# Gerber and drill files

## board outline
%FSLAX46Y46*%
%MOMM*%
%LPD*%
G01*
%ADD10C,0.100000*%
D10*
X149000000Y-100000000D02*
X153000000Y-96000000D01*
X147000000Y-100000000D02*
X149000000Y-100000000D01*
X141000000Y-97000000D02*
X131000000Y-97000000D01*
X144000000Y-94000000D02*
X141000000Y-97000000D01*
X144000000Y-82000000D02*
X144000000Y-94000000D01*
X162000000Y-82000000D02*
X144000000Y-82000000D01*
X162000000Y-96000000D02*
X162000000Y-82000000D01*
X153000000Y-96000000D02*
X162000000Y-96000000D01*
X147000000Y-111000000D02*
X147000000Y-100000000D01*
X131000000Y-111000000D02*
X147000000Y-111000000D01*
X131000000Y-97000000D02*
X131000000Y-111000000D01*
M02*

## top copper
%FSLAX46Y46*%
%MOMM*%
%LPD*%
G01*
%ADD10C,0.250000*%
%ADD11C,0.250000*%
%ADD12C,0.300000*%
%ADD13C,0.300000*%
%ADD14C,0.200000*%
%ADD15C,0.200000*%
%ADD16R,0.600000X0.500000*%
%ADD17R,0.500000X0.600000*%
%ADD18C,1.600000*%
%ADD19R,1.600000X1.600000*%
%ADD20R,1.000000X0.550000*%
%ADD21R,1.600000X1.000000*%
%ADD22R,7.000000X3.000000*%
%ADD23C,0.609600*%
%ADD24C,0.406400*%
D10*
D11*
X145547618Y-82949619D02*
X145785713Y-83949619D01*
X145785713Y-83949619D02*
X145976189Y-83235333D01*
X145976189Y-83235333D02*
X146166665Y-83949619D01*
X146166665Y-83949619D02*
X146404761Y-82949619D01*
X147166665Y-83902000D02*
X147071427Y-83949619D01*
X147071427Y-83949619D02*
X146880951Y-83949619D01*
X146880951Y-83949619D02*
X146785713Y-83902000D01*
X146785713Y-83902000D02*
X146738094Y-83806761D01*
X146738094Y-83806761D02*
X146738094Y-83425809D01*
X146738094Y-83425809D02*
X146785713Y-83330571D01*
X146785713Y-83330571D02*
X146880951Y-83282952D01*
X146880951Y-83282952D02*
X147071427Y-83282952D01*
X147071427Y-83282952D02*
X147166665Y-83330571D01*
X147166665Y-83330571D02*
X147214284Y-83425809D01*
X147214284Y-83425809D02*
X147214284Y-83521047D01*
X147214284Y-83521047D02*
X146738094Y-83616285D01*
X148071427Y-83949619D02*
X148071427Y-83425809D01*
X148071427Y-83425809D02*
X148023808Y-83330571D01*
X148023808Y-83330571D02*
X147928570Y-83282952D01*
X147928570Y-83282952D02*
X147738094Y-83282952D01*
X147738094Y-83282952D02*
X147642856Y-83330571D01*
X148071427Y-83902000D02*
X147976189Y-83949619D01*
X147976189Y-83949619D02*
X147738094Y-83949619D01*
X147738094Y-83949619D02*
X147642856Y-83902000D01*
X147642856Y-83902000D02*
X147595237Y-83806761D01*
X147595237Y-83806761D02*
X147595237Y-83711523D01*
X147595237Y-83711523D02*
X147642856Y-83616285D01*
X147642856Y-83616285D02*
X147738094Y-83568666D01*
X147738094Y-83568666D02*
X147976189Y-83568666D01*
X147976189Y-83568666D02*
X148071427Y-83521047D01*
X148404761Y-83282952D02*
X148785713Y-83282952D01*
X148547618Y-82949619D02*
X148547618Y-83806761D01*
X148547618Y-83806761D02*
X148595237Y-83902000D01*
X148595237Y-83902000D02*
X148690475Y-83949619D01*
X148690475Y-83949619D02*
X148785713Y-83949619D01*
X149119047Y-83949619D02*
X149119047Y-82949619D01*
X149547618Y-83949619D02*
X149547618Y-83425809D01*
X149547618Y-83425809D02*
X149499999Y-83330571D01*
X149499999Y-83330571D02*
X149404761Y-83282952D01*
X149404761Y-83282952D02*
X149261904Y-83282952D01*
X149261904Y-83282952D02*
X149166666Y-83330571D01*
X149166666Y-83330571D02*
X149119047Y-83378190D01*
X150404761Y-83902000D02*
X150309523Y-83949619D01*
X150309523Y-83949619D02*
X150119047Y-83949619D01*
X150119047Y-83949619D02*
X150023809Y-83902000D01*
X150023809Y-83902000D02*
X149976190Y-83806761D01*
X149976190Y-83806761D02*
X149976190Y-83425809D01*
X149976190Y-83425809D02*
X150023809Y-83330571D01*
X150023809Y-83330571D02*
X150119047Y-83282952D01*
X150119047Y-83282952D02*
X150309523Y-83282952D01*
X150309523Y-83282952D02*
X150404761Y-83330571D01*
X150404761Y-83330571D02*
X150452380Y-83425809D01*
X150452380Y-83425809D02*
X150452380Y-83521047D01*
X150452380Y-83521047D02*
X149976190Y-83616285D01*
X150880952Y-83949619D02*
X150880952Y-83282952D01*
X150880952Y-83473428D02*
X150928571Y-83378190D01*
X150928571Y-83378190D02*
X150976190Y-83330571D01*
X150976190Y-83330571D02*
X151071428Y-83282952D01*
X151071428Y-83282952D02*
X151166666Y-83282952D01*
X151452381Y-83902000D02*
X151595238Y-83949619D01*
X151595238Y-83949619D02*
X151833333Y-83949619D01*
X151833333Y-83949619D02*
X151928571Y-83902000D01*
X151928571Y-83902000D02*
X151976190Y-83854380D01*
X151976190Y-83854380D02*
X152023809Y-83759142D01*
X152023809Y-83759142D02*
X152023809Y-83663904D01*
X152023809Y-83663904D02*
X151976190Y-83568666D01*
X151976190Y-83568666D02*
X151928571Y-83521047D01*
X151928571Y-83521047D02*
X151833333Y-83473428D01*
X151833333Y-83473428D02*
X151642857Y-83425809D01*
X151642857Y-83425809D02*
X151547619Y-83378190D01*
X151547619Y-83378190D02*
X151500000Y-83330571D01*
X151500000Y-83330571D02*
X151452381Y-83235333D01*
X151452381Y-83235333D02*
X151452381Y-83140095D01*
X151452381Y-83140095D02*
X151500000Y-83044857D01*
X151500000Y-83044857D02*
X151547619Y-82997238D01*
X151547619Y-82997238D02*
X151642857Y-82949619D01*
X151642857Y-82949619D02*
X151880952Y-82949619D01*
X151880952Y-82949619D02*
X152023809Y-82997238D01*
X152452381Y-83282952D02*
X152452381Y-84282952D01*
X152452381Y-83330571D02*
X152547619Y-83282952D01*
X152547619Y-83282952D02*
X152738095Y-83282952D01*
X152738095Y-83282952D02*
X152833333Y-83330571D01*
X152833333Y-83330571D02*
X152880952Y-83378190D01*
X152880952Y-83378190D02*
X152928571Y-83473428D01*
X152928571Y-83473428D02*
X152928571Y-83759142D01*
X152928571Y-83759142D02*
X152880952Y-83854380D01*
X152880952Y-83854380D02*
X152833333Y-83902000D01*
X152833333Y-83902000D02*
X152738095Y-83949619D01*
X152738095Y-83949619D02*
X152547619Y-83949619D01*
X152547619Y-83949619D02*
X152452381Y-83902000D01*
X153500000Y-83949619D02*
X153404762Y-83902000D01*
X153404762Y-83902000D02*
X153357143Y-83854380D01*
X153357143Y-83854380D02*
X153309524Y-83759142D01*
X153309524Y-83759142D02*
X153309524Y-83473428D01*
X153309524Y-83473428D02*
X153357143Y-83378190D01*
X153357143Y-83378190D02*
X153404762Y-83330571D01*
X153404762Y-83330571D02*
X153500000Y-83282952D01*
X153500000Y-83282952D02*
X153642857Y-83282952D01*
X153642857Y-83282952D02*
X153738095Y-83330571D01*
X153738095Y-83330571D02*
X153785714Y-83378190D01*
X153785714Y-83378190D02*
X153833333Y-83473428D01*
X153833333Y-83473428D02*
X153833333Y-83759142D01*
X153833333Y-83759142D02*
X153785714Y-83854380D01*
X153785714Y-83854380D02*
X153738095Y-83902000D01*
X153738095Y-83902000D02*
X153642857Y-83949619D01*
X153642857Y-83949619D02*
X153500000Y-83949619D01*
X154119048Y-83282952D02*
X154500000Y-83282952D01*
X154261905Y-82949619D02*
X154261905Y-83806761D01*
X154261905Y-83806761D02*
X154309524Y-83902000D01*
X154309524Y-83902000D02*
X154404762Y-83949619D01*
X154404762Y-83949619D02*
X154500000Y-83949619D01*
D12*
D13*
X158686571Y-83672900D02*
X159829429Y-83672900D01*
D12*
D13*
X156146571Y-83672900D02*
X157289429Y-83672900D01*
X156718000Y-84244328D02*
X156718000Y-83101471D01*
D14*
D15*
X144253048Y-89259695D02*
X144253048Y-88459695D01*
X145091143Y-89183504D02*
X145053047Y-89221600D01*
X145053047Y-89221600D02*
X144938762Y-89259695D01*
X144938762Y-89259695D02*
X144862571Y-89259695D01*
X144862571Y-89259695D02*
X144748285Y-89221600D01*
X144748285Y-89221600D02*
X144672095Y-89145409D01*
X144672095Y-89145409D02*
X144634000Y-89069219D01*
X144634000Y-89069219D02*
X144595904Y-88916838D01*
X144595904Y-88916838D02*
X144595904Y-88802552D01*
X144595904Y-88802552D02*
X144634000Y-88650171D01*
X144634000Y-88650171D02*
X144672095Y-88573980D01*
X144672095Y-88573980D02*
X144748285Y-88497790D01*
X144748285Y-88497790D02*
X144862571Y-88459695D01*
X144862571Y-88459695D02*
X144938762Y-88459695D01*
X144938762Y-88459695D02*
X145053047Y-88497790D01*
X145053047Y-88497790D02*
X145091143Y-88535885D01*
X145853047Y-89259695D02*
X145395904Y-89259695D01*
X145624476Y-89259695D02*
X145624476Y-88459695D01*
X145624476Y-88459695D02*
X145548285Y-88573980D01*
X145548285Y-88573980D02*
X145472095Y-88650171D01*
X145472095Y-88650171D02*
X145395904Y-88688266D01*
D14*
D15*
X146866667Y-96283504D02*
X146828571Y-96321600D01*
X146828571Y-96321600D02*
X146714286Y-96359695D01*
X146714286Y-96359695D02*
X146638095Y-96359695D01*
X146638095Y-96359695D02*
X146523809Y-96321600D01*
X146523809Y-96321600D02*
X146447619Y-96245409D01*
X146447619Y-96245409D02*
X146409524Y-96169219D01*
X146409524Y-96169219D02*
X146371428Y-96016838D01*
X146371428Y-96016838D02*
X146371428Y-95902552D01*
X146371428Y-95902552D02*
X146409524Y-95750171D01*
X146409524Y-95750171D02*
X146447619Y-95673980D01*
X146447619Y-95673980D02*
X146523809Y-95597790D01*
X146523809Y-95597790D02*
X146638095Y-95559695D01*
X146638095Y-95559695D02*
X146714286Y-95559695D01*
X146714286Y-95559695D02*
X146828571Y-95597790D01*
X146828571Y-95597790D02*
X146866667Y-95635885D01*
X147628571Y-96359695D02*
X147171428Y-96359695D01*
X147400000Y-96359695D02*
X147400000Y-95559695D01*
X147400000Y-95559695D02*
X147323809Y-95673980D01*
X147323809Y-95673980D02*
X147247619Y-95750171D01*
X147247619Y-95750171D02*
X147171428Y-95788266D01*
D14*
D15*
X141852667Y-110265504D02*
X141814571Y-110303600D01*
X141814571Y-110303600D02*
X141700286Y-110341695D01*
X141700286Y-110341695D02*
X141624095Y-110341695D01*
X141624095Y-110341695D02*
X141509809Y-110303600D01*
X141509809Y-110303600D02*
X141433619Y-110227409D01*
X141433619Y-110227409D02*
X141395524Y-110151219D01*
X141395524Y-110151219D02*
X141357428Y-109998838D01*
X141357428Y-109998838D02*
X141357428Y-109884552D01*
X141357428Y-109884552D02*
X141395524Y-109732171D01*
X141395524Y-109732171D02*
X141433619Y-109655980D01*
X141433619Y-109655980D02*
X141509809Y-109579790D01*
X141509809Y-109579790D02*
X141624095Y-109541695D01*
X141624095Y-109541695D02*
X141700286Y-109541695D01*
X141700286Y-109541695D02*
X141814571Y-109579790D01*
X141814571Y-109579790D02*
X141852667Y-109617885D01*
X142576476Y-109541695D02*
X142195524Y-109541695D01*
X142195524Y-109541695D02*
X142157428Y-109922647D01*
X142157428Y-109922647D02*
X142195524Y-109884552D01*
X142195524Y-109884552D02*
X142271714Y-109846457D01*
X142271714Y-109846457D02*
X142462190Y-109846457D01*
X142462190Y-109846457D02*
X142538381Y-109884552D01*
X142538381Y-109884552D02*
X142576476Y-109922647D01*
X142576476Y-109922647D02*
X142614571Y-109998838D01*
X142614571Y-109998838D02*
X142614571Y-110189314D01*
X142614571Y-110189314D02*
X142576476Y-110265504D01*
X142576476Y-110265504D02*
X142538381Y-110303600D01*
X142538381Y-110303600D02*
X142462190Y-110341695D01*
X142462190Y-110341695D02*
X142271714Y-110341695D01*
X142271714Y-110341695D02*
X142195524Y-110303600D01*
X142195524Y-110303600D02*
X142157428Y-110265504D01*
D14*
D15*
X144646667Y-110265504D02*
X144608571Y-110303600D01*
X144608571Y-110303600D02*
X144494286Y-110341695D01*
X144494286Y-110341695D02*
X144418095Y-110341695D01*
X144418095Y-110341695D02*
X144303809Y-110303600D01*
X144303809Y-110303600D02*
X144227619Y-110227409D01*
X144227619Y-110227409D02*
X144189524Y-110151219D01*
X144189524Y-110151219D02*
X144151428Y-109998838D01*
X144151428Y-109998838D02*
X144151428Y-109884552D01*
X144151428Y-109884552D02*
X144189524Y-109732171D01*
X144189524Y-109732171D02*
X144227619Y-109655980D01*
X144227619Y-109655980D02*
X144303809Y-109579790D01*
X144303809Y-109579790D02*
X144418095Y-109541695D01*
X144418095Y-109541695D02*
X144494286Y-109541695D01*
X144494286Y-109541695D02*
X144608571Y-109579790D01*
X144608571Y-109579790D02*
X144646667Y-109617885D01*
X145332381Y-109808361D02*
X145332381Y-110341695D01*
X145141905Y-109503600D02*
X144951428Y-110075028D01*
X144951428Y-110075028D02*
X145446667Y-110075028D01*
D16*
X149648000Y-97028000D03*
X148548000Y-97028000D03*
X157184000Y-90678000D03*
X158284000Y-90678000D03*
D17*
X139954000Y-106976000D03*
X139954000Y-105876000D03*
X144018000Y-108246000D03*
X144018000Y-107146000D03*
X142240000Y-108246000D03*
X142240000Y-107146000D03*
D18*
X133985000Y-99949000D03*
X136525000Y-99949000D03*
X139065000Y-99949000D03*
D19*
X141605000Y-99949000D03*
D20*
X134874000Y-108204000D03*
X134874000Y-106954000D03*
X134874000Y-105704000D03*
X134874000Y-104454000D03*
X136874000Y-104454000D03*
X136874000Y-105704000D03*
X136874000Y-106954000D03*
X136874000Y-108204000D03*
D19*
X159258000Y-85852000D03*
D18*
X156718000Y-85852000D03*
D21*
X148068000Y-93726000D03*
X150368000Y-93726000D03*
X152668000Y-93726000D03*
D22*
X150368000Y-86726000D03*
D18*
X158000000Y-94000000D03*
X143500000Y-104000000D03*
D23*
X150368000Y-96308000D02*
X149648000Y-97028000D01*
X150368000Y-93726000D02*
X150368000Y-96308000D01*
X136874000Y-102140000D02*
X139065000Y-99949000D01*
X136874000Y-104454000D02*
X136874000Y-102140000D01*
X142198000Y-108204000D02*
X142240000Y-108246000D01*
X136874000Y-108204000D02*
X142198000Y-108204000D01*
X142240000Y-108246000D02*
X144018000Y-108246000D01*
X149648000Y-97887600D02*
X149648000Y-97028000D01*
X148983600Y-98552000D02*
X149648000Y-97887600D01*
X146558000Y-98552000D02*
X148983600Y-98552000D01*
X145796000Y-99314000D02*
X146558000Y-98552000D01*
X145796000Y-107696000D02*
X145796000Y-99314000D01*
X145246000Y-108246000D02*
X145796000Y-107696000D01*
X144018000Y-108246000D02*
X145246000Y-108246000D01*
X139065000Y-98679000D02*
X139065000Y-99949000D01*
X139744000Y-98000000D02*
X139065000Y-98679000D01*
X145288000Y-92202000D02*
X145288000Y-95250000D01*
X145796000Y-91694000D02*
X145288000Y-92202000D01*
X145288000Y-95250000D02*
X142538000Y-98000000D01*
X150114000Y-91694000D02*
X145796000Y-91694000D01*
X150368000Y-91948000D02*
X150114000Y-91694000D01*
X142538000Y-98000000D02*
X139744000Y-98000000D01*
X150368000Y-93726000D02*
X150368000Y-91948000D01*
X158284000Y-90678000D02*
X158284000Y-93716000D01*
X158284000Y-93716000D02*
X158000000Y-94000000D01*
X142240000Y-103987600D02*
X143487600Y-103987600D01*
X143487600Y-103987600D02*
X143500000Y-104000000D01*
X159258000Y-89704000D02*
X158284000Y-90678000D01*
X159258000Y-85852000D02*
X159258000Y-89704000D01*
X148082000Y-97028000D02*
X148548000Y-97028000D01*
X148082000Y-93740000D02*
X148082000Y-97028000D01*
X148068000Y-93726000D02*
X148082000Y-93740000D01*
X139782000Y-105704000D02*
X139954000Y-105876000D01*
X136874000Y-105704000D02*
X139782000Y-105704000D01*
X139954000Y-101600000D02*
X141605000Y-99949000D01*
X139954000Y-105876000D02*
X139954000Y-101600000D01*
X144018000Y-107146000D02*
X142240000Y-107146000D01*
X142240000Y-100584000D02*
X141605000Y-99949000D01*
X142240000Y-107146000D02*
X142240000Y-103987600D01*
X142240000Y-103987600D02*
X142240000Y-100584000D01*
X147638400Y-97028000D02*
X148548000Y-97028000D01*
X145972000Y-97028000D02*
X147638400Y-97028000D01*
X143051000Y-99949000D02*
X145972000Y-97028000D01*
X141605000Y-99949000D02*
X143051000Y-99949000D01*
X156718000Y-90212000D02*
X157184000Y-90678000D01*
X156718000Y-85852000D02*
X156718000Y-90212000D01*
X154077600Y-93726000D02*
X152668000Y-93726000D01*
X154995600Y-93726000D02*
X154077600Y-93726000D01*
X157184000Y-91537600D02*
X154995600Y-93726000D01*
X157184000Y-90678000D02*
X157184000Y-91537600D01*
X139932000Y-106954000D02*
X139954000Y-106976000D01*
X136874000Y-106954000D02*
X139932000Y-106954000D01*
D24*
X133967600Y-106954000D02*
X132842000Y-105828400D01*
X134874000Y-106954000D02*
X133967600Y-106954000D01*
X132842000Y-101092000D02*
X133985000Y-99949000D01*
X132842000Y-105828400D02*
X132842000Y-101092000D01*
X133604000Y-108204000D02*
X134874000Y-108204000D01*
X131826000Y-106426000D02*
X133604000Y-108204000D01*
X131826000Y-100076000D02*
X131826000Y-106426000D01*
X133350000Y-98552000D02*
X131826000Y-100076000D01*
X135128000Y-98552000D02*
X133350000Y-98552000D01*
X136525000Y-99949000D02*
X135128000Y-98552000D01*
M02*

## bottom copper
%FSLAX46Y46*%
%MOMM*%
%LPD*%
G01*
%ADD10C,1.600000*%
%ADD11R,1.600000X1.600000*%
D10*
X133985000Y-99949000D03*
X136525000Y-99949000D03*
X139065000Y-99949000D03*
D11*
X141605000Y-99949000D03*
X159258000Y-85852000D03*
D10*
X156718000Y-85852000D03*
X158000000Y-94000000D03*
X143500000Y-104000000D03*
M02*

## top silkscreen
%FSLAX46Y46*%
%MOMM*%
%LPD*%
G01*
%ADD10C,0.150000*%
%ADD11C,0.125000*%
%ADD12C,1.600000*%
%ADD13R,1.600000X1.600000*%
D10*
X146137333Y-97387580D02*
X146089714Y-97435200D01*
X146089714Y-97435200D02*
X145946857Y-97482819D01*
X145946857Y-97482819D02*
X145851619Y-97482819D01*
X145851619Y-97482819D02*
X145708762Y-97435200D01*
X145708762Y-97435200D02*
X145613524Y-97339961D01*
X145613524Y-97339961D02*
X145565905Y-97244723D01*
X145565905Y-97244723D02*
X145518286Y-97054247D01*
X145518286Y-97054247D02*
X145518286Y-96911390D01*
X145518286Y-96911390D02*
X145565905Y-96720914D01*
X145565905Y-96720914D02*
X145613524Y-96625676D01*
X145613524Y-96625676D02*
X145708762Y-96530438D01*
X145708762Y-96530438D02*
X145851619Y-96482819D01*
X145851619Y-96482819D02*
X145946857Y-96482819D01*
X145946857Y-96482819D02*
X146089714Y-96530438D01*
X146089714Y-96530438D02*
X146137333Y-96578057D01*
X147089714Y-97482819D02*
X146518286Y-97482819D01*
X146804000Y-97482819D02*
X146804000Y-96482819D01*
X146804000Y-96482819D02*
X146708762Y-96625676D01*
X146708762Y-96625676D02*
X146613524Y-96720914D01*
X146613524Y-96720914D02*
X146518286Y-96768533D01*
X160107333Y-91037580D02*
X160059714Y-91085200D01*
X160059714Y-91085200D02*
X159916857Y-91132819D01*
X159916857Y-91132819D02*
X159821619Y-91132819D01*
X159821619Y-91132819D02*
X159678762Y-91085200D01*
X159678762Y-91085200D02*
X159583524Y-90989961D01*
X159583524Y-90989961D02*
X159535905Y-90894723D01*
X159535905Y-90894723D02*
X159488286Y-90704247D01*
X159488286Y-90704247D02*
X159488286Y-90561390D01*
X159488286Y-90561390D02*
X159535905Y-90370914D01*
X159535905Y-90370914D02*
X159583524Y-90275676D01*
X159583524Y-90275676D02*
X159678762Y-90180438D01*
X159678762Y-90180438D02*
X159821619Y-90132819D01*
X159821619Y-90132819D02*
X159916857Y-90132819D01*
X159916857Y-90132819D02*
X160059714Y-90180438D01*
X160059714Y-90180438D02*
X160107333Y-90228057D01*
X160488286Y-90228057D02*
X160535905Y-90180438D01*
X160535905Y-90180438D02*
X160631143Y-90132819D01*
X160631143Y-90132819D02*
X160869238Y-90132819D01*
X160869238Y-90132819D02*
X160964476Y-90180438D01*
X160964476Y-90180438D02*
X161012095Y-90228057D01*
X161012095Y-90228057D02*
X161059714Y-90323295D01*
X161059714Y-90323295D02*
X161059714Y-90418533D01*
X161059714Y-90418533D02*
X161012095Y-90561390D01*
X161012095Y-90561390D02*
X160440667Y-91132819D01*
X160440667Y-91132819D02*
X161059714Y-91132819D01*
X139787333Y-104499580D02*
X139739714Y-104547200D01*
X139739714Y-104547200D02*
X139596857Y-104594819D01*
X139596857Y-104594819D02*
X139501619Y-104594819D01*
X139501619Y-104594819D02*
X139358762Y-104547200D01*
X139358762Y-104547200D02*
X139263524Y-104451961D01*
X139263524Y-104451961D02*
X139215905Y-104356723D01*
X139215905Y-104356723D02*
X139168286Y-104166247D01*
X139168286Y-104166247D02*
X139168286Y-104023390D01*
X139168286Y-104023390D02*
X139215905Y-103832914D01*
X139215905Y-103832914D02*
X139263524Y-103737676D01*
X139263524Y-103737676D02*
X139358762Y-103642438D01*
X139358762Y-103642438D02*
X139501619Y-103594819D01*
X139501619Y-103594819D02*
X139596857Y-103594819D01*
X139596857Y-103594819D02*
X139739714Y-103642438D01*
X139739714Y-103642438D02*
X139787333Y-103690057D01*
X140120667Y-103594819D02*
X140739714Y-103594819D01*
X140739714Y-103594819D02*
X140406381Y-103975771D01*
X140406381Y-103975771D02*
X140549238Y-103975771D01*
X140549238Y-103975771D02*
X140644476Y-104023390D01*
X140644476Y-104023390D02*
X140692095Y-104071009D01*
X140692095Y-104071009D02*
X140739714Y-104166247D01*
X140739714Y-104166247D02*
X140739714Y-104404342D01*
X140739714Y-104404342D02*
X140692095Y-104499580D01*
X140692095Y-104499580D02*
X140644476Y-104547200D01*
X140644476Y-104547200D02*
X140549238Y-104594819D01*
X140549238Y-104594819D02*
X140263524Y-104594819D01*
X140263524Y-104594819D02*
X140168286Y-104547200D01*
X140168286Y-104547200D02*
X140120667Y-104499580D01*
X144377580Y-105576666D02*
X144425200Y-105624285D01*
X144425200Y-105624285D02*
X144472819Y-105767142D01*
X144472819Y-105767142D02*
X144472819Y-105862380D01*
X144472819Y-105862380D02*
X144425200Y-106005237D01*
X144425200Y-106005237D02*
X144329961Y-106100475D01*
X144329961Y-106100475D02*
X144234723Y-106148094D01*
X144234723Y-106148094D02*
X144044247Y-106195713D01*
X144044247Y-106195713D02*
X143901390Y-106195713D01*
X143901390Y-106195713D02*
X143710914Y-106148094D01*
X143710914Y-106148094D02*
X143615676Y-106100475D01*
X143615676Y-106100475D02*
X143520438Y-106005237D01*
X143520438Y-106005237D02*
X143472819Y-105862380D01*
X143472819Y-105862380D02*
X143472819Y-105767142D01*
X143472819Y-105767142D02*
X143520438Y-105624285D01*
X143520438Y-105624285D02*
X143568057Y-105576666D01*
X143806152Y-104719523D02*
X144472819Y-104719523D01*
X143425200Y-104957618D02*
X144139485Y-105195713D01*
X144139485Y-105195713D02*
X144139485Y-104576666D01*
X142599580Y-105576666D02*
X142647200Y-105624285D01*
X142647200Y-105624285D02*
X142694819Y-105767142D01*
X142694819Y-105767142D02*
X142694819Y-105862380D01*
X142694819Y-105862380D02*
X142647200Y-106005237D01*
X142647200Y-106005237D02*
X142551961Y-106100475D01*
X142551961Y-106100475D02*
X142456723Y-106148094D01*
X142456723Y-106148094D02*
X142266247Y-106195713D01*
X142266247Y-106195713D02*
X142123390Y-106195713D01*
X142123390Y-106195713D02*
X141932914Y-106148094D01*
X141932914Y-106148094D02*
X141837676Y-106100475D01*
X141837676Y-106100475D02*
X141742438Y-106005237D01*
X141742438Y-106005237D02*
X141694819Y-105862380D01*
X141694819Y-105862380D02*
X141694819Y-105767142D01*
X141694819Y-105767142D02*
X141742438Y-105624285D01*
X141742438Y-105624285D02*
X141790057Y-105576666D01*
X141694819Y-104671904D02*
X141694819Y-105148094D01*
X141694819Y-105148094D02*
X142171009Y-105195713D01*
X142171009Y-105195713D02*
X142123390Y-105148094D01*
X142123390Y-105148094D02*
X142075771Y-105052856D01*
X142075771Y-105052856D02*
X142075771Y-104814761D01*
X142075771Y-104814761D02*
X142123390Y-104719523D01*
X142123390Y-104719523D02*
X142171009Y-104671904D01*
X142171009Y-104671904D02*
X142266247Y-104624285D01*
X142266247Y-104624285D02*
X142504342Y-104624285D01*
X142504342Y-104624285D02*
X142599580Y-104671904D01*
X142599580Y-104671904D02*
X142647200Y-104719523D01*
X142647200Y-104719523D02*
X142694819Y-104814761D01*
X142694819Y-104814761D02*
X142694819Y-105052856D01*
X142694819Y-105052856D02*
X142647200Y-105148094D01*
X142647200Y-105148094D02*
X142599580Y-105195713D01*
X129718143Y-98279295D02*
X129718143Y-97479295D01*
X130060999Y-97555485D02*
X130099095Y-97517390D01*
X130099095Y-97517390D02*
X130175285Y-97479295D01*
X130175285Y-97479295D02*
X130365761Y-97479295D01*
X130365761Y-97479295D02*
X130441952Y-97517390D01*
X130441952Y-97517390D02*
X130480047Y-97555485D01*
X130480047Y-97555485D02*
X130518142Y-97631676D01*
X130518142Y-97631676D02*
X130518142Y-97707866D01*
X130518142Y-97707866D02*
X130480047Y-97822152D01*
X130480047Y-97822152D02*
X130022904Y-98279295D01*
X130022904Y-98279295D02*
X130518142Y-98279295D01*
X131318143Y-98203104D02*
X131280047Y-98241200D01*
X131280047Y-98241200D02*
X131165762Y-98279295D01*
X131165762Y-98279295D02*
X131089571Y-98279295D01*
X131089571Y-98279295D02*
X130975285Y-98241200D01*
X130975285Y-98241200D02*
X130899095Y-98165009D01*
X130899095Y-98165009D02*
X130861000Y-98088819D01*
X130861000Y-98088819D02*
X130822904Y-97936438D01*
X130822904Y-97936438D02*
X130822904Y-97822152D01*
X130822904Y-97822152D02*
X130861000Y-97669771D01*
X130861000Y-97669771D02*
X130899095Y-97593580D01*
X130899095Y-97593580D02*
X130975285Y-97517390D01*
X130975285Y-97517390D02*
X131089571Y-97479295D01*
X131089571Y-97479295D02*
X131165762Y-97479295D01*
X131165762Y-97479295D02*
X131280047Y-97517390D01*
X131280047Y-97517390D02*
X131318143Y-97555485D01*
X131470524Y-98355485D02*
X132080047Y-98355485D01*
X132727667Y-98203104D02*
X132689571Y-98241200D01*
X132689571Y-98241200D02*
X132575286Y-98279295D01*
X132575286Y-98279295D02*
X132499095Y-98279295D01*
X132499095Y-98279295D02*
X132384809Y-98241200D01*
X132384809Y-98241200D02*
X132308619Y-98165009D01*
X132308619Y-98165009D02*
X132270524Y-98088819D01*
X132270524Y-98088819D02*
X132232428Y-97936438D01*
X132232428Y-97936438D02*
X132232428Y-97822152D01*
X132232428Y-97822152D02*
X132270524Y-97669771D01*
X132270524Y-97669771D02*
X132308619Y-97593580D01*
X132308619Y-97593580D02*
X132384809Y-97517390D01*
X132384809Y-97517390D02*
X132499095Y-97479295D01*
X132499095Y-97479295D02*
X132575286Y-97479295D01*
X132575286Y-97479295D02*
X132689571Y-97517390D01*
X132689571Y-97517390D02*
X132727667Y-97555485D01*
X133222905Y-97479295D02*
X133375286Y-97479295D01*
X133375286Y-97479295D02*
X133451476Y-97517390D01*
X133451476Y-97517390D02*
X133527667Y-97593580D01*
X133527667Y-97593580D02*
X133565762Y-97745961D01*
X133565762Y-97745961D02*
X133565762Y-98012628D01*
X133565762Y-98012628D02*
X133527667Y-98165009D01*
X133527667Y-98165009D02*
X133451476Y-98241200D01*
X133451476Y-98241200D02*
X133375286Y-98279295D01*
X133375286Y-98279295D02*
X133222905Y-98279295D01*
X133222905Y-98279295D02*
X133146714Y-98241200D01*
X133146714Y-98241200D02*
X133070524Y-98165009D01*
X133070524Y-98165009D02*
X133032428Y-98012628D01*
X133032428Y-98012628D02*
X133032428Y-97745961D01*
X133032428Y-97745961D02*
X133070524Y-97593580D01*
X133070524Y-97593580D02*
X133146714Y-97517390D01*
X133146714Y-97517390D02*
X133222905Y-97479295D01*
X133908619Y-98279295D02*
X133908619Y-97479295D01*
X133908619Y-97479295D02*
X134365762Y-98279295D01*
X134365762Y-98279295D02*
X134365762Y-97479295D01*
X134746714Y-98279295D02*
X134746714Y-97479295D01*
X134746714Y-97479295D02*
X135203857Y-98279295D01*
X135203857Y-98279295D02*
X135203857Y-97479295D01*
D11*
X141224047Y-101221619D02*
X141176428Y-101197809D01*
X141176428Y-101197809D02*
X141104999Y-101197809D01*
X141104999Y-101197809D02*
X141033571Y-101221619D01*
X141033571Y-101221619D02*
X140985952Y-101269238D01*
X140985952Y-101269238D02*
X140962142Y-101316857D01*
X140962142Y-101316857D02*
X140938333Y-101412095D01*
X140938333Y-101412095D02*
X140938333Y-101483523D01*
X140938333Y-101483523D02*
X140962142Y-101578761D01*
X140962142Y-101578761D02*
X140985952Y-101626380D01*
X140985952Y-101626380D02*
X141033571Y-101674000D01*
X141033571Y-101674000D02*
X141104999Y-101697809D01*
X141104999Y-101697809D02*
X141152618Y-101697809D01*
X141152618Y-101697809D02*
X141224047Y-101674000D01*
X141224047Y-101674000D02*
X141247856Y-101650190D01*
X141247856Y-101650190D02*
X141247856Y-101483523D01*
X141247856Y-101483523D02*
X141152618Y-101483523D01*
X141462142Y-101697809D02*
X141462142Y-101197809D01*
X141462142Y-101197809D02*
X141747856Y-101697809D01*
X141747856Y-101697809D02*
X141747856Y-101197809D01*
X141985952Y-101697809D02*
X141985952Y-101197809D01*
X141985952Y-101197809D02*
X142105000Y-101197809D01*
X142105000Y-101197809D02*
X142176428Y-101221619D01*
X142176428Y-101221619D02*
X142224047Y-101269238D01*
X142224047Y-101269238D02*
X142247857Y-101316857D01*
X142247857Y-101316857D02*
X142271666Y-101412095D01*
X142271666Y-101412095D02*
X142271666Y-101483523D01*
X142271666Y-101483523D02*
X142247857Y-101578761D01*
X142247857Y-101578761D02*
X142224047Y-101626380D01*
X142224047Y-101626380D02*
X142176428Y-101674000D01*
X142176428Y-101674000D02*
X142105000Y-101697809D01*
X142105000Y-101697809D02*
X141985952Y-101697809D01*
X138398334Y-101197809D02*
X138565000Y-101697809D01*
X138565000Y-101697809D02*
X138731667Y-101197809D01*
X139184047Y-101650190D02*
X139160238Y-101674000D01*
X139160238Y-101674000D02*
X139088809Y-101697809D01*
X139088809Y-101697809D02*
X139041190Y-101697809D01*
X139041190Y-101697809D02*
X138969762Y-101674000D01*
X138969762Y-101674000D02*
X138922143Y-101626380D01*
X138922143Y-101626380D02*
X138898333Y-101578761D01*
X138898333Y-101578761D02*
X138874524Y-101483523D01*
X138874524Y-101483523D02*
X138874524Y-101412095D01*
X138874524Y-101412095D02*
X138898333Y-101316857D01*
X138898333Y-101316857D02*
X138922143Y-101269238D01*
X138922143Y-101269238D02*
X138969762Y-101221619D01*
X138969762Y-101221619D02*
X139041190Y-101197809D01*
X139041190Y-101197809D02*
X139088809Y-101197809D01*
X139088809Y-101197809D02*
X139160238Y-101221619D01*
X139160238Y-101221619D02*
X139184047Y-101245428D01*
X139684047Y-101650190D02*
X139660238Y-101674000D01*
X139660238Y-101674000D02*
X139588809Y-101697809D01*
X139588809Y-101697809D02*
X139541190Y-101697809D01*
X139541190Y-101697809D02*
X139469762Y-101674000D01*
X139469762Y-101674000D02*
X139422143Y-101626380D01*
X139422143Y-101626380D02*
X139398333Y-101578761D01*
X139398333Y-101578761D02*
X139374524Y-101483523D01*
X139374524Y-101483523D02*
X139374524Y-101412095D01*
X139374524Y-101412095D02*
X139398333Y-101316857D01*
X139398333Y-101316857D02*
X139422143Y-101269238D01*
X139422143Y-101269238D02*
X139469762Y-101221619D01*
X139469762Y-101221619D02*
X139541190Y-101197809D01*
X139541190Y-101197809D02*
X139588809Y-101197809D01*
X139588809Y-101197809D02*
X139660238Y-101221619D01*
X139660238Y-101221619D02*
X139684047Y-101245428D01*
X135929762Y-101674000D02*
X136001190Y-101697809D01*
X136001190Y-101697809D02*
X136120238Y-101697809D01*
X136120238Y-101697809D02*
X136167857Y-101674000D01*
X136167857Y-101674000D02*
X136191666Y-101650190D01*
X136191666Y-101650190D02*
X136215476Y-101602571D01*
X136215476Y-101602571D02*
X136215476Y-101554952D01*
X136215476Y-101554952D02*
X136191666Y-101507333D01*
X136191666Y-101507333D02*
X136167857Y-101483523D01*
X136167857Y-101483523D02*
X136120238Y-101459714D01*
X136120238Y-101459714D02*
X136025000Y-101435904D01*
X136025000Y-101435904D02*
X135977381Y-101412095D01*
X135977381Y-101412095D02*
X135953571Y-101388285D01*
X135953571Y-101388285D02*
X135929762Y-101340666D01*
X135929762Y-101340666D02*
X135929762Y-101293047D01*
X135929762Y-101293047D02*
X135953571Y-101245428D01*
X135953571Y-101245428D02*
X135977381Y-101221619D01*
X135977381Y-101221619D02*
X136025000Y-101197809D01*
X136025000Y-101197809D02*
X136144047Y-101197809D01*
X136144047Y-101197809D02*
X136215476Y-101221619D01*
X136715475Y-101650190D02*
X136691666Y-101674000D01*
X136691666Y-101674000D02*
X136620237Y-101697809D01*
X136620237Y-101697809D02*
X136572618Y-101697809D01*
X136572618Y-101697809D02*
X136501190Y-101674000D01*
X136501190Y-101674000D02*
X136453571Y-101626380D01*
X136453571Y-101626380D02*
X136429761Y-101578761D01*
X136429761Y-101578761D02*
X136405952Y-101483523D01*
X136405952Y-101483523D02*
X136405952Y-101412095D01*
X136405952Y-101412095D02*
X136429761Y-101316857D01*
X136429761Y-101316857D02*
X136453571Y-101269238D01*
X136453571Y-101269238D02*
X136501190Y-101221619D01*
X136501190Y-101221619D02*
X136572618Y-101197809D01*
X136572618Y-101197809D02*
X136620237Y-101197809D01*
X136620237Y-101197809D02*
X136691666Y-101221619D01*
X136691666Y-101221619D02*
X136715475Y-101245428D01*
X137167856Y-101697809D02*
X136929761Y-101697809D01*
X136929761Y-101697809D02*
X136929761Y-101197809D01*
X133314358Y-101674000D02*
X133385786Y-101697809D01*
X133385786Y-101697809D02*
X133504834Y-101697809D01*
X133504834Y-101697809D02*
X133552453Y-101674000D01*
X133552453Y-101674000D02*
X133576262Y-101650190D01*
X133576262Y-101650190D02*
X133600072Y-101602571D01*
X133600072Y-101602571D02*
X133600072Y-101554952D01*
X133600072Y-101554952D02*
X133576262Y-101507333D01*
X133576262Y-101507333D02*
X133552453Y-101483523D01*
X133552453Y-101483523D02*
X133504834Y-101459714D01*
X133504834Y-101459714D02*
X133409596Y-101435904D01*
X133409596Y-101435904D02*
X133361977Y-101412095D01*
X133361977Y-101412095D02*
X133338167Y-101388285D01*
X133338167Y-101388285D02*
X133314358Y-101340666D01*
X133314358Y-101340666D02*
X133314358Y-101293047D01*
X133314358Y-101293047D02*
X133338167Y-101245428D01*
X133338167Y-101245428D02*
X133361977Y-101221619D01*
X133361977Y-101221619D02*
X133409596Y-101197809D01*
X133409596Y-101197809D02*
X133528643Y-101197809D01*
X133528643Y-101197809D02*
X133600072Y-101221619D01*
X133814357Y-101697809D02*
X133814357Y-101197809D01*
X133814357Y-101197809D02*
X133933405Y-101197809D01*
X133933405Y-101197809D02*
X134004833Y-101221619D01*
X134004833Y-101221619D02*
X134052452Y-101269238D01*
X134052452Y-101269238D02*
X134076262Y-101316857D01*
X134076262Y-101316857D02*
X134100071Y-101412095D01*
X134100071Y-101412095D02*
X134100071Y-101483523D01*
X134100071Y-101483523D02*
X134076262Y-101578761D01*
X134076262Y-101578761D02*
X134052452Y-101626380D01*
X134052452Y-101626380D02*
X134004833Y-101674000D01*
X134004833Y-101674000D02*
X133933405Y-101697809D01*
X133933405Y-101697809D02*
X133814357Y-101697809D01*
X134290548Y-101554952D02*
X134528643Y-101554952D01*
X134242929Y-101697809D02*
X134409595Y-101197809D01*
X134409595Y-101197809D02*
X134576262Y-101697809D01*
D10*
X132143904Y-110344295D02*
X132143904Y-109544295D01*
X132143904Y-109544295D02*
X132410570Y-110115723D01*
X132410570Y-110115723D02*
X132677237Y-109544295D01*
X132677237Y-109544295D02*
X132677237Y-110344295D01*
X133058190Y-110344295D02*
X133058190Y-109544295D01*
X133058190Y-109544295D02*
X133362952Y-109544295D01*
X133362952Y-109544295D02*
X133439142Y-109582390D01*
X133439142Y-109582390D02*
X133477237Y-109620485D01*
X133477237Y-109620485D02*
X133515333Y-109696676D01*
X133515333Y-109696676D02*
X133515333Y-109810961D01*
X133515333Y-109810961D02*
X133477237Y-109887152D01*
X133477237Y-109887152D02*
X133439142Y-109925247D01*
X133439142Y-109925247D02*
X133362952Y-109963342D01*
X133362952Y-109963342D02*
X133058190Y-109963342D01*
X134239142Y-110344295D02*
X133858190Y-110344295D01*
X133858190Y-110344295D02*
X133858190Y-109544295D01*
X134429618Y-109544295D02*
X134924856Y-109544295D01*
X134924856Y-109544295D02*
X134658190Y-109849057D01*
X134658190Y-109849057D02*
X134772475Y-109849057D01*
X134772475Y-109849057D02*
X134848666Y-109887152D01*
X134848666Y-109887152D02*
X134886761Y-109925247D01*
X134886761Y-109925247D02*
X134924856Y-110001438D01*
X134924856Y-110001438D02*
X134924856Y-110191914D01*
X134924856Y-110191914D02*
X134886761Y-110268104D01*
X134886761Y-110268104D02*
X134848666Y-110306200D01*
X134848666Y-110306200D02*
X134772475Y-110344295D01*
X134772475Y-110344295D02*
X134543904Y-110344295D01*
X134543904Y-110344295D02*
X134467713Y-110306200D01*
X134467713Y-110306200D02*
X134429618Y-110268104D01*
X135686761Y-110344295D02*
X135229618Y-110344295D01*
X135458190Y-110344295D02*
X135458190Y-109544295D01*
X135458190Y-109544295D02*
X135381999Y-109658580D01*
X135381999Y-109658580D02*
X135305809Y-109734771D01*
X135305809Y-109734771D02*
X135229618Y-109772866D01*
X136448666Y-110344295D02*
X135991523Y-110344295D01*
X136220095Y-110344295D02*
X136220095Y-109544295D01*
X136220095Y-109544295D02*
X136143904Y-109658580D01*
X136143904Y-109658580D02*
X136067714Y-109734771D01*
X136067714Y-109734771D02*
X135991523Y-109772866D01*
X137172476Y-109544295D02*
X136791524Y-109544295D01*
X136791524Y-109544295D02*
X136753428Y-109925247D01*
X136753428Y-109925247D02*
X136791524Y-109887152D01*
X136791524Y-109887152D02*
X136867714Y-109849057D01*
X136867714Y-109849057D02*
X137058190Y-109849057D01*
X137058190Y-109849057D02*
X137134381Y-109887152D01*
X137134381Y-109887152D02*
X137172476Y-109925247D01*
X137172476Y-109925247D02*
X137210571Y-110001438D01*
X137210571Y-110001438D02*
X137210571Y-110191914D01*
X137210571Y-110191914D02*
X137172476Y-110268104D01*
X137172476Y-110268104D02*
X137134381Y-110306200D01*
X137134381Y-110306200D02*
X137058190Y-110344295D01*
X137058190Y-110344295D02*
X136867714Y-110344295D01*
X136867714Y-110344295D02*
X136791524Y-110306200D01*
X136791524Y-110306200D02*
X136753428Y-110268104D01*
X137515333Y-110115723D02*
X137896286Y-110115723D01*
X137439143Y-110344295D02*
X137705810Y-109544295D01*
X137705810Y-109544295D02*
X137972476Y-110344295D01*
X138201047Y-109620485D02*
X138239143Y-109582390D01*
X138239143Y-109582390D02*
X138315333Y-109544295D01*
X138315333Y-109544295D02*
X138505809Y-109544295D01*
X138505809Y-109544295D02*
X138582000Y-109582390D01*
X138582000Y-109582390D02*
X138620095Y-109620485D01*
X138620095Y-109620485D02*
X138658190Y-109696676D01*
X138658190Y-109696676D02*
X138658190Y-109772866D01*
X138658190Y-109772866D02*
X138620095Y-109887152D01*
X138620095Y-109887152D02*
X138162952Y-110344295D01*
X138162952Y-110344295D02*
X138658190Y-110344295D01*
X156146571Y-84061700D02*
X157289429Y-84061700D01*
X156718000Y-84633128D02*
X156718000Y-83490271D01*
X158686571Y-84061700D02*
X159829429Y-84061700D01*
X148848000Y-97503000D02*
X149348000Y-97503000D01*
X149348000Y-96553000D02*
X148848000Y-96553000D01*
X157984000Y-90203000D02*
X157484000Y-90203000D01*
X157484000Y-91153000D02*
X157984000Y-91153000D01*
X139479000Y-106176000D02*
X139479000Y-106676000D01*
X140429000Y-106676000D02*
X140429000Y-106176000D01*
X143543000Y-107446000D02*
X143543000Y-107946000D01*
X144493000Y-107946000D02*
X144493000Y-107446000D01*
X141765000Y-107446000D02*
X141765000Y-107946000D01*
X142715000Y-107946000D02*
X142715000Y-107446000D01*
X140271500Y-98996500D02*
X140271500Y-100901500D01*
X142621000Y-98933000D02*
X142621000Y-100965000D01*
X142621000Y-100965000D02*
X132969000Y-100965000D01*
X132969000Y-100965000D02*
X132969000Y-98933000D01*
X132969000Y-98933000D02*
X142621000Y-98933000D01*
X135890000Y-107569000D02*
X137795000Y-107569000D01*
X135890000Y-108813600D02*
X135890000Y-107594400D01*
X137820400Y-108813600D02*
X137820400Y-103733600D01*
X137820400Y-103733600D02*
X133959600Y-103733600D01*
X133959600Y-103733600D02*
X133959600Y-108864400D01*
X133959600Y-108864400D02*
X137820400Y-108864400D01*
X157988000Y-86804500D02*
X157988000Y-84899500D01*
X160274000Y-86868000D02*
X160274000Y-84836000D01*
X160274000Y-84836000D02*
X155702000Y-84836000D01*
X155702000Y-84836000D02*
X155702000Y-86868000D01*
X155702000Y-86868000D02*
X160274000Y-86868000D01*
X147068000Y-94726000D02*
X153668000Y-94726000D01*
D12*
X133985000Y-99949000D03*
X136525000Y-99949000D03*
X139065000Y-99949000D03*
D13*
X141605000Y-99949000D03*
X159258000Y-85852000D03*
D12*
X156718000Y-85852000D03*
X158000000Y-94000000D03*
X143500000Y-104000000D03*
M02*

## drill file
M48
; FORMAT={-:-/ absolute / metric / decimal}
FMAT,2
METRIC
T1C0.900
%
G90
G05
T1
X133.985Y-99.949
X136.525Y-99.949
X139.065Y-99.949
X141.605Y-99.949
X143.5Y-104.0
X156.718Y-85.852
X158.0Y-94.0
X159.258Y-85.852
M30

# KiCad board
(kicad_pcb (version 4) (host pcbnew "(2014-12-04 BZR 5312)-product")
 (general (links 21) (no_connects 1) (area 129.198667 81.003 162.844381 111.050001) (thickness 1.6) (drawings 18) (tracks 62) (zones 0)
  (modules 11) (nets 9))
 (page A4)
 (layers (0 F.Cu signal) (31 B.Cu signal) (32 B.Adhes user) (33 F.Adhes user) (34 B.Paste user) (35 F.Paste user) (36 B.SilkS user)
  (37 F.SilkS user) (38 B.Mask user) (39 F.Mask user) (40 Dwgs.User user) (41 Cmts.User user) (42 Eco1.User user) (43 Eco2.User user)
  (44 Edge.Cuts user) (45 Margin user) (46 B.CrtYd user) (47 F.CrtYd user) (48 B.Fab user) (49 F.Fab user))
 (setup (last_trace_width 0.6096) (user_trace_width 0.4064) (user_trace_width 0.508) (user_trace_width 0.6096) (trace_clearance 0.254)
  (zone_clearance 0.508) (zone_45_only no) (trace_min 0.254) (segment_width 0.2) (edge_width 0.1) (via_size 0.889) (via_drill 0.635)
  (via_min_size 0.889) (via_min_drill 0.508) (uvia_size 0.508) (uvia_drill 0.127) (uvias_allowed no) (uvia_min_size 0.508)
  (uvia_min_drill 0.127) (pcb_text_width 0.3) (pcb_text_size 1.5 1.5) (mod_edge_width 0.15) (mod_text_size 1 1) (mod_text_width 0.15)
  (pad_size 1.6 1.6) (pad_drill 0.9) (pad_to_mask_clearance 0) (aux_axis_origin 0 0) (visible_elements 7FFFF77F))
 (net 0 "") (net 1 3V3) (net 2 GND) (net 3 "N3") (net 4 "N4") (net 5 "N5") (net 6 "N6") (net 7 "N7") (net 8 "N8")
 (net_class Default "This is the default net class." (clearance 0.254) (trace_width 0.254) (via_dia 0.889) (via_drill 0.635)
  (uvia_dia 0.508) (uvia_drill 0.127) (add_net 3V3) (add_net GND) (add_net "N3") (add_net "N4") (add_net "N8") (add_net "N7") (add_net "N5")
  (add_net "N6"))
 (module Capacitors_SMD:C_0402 (layer F.Cu) (at 149.098 97.028 180)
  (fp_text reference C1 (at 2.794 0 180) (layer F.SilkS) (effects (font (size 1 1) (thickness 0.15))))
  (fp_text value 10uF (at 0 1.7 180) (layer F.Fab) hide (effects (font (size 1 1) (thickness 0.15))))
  (fp_line (start 0.25 -0.475) (end -0.25 -0.475) (layer F.SilkS) (width 0.15))
  (fp_line (start -0.25 0.475) (end 0.25 0.475) (layer F.SilkS) (width 0.15))
  (pad 1 smd rect (at -0.55 0 180) (size 0.6 0.5) (layers F.Cu F.Paste F.Mask) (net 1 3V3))
  (pad 2 smd rect (at 0.55 0 180) (size 0.6 0.5) (layers F.Cu F.Paste F.Mask) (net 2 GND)))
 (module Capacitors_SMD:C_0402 (layer F.Cu) (at 157.734 90.678)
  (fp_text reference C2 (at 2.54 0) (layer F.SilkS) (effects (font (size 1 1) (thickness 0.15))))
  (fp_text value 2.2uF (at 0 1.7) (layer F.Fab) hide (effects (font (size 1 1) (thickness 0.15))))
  (fp_line (start 0.25 -0.475) (end -0.25 -0.475) (layer F.SilkS) (width 0.15))
  (fp_line (start -0.25 0.475) (end 0.25 0.475) (layer F.SilkS) (width 0.15))
  (pad 1 smd rect (at -0.55 0) (size 0.6 0.5) (layers F.Cu F.Paste F.Mask) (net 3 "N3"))
  (pad 2 smd rect (at 0.55 0) (size 0.6 0.5) (layers F.Cu F.Paste F.Mask) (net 2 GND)))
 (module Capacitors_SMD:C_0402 (layer F.Cu) (at 139.954 106.426 90)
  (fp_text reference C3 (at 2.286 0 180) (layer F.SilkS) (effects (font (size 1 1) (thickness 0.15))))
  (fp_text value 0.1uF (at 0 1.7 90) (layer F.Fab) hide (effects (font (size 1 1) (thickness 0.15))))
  (fp_line (start 0.25 -0.475) (end -0.25 -0.475) (layer F.SilkS) (width 0.15))
  (fp_line (start -0.25 0.475) (end 0.25 0.475) (layer F.SilkS) (width 0.15))
  (pad 1 smd rect (at -0.55 0 90) (size 0.6 0.5) (layers F.Cu F.Paste F.Mask) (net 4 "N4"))
  (pad 2 smd rect (at 0.55 0 90) (size 0.6 0.5) (layers F.Cu F.Paste F.Mask) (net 2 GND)))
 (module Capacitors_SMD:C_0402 (layer F.Cu) (at 144.018 107.696 90)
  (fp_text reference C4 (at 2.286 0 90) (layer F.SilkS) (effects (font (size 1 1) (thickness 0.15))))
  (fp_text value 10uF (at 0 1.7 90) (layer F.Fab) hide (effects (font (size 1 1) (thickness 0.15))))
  (fp_line (start 0.25 -0.475) (end -0.25 -0.475) (layer F.SilkS) (width 0.15))
  (fp_line (start -0.25 0.475) (end 0.25 0.475) (layer F.SilkS) (width 0.15))
  (pad 1 smd rect (at -0.55 0 90) (size 0.6 0.5) (layers F.Cu F.Paste F.Mask) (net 1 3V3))
  (pad 2 smd rect (at 0.55 0 90) (size 0.6 0.5) (layers F.Cu F.Paste F.Mask) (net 2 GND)))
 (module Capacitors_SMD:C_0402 (layer F.Cu) (at 142.24 107.696 90)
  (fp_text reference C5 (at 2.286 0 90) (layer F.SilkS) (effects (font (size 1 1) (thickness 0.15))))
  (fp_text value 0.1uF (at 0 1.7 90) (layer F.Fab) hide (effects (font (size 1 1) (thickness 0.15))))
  (fp_line (start 0.25 -0.475) (end -0.25 -0.475) (layer F.SilkS) (width 0.15))
  (fp_line (start -0.25 0.475) (end 0.25 0.475) (layer F.SilkS) (width 0.15))
  (pad 1 smd rect (at -0.55 0 90) (size 0.6 0.5) (layers F.Cu F.Paste F.Mask) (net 1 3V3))
  (pad 2 smd rect (at 0.55 0 90) (size 0.6 0.5) (layers F.Cu F.Paste F.Mask) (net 2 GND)))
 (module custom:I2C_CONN (layer F.Cu) (at 139.065 99.949)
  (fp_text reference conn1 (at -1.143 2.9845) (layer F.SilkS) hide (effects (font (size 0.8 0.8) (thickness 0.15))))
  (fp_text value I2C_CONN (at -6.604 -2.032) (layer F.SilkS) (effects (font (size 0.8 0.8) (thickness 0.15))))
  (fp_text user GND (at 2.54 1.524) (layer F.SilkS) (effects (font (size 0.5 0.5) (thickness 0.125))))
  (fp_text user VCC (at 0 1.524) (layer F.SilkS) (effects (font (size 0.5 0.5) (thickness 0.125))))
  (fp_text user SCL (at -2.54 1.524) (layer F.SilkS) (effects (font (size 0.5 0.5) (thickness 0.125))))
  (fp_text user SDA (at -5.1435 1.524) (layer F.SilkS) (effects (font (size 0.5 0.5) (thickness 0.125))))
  (fp_line (start 1.2065 -0.9525) (end 1.2065 0.9525) (layer F.SilkS) (width 0.15))
  (fp_line (start 3.556 -1.016) (end 3.556 1.016) (layer F.SilkS) (width 0.15))
  (fp_line (start 3.556 1.016) (end -6.096 1.016) (layer F.SilkS) (width 0.15))
  (fp_line (start -6.096 1.016) (end -6.096 -1.016) (layer F.SilkS) (width 0.15))
  (fp_line (start -6.096 -1.016) (end 3.556 -1.016) (layer F.SilkS) (width 0.15))
  (pad 1 thru_hole circle (at -5.08 0) (size 1.6 1.6) (drill 0.9) (layers *.Cu *.Mask F.SilkS) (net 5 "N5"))
  (pad 2 thru_hole circle (at -2.54 0) (size 1.6 1.6) (drill 0.9) (layers *.Cu *.Mask F.SilkS) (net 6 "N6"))
  (pad 3 thru_hole circle (at 0 0) (size 1.6 1.6) (drill 0.9) (layers *.Cu *.Mask F.SilkS) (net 1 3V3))
  (pad 4 thru_hole rect (at 2.54 0) (size 1.6 1.6) (drill 0.9) (layers *.Cu *.Mask F.SilkS) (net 2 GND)))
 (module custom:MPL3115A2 (layer F.Cu) (at 134.874 108.204 180)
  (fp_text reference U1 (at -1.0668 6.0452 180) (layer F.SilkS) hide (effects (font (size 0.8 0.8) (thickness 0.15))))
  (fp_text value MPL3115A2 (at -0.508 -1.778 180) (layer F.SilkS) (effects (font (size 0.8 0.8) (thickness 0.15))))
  (fp_line (start -1.016 0.635) (end -2.921 0.635) (layer F.SilkS) (width 0.15))
  (fp_line (start -1.016 -0.6096) (end -1.016 0.6096) (layer F.SilkS) (width 0.15))
  (fp_line (start -2.9464 -0.6096) (end -2.9464 4.4704) (layer F.SilkS) (width 0.15))
  (fp_line (start -2.9464 4.4704) (end 0.9144 4.4704) (layer F.SilkS) (width 0.15))
  (fp_line (start 0.9144 4.4704) (end 0.9144 -0.6604) (layer F.SilkS) (width 0.15))
  (fp_line (start 0.9144 -0.6604) (end -2.9464 -0.6604) (layer F.SilkS) (width 0.15))
  (pad 8 smd rect (at 0 0 180) (size 1 0.55) (layers F.Cu F.Paste F.Mask) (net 6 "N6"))
  (pad 7 smd rect (at 0 1.25 180) (size 1 0.55) (layers F.Cu F.Paste F.Mask) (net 5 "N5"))
  (pad 6 smd rect (at 0 2.5 180) (size 1 0.55) (layers F.Cu F.Paste F.Mask) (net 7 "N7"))
  (pad 5 smd rect (at 0 3.75 180) (size 1 0.55) (layers F.Cu F.Paste F.Mask) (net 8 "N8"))
  (pad 4 smd rect (at -2 3.75 180) (size 1 0.55) (layers F.Cu F.Paste F.Mask) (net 1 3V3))
  (pad 3 smd rect (at -2 2.5 180) (size 1 0.55) (layers F.Cu F.Paste F.Mask) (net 2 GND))
  (pad 2 smd rect (at -2 1.25 180) (size 1 0.55) (layers F.Cu F.Paste F.Mask) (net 4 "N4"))
  (pad 1 smd rect (at -2 0 180) (size 1 0.55) (layers F.Cu F.Paste F.Mask) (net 1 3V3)))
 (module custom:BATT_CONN (layer F.Cu) (at 156.718 85.852 180)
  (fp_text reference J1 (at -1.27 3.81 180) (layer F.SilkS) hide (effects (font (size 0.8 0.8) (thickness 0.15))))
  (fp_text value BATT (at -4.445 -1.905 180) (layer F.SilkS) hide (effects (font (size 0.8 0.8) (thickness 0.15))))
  (fp_line (start -1.27 -0.9525) (end -1.27 0.9525) (layer F.SilkS) (width 0.15))
  (fp_line (start -3.556 -1.016) (end -3.556 1.016) (layer F.SilkS) (width 0.15))
  (fp_line (start -3.556 1.016) (end 1.016 1.016) (layer F.SilkS) (width 0.15))
  (fp_line (start 1.016 1.016) (end 1.016 -1.016) (layer F.SilkS) (width 0.15))
  (fp_line (start 1.016 -1.016) (end -3.556 -1.016) (layer F.SilkS) (width 0.15))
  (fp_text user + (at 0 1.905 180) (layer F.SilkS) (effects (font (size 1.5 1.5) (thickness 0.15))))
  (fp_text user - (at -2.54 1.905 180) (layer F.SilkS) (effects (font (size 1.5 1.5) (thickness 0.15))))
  (pad 1 thru_hole rect (at -2.54 0 180) (size 1.6 1.6) (drill 0.9) (layers *.Cu *.Mask F.SilkS) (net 2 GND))
  (pad 2 thru_hole circle (at 0 0 180) (size 1.6 1.6) (drill 0.9) (layers *.Cu *.Mask F.SilkS) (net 3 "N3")))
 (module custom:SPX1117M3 (layer F.Cu) (at 150.368 93.726)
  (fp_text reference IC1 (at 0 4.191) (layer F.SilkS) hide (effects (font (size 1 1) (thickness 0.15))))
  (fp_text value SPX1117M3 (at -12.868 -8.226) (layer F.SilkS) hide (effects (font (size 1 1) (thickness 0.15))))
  (fp_line (start -3.3 1) (end 3.3 1) (layer F.SilkS) (width 0.15))
  (pad 1 smd rect (at -2.3 0) (size 1.6 1) (layers F.Cu F.Paste F.Mask) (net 2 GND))
  (pad 2 smd rect (at 0 0) (size 1.6 1) (layers F.Cu F.Paste F.Mask) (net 1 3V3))
  (pad 3 smd rect (at 2.3 0) (size 1.6 1) (layers F.Cu F.Paste F.Mask) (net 3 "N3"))
  (pad "" smd rect (at 0 -7) (size 7 3) (layers F.Cu F.Paste F.Mask)))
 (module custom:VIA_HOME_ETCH (layer F.Cu) (at 158 94)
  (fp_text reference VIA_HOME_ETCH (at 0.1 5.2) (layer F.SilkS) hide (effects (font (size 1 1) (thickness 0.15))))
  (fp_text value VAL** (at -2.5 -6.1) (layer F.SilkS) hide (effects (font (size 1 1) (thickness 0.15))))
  (pad 1 thru_hole circle (at 0 0) (size 1.6 1.6) (drill 0.9) (layers *.Cu *.Mask F.SilkS) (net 2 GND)))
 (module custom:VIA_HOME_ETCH (layer F.Cu) (at 143.5 104)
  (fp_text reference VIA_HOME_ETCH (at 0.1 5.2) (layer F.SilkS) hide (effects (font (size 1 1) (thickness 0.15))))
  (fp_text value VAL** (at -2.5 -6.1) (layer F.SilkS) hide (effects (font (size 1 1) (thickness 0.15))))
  (pad 1 thru_hole circle (at 0 0) (size 1.6 1.6) (drill 0.9) (layers *.Cu *.Mask F.SilkS) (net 2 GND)))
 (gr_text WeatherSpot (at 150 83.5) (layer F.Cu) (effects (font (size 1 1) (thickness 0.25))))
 (gr_line (start 149 100) (end 153 96) (angle 90) (layer Edge.Cuts) (width 0.1))
 (gr_line (start 147 100) (end 149 100) (angle 90) (layer Edge.Cuts) (width 0.1))
 (gr_line (start 141 97) (end 131 97) (angle 90) (layer Edge.Cuts) (width 0.1))
 (gr_line (start 144 94) (end 141 97) (angle 90) (layer Edge.Cuts) (width 0.1))
 (gr_line (start 144 82) (end 144 94) (angle 90) (layer Edge.Cuts) (width 0.1))
 (gr_line (start 162 82) (end 144 82) (angle 90) (layer Edge.Cuts) (width 0.1))
 (gr_line (start 162 96) (end 162 82) (angle 90) (layer Edge.Cuts) (width 0.1))
 (gr_line (start 153 96) (end 162 96) (angle 90) (layer Edge.Cuts) (width 0.1))
 (gr_line (start 147 111) (end 147 100) (angle 90) (layer Edge.Cuts) (width 0.1))
 (gr_line (start 131 111) (end 147 111) (angle 90) (layer Edge.Cuts) (width 0.1))
 (gr_line (start 131 97) (end 131 111) (angle 90) (layer Edge.Cuts) (width 0.1))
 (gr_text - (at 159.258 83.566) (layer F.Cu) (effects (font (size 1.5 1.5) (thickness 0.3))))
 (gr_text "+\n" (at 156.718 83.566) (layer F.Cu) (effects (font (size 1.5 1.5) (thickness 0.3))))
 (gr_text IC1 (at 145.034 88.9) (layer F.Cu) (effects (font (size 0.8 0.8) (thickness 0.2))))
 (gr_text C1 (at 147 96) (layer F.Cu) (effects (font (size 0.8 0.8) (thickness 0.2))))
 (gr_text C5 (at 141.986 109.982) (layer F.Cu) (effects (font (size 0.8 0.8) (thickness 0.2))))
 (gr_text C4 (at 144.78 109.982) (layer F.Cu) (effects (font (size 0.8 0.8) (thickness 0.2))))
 (segment (start 150.368 96.308) (end 149.648 97.028) (width 0.6096) (layer F.Cu) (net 1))
 (segment (start 150.368 93.726) (end 150.368 96.308) (width 0.6096) (layer F.Cu) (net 1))
 (segment (start 136.874 102.14) (end 139.065 99.949) (width 0.6096) (layer F.Cu) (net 1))
 (segment (start 136.874 104.454) (end 136.874 102.14) (width 0.6096) (layer F.Cu) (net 1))
 (segment (start 142.198 108.204) (end 142.24 108.246) (width 0.6096) (layer F.Cu) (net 1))
 (segment (start 136.874 108.204) (end 142.198 108.204) (width 0.6096) (layer F.Cu) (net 1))
 (segment (start 142.24 108.246) (end 144.018 108.246) (width 0.6096) (layer F.Cu) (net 1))
 (segment (start 149.648 97.8876) (end 149.648 97.028) (width 0.6096) (layer F.Cu) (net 1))
 (segment (start 148.9836 98.552) (end 149.648 97.8876) (width 0.6096) (layer F.Cu) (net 1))
 (segment (start 146.558 98.552) (end 148.9836 98.552) (width 0.6096) (layer F.Cu) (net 1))
 (segment (start 145.796 99.314) (end 146.558 98.552) (width 0.6096) (layer F.Cu) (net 1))
 (segment (start 145.796 107.696) (end 145.796 99.314) (width 0.6096) (layer F.Cu) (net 1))
 (segment (start 145.246 108.246) (end 145.796 107.696) (width 0.6096) (layer F.Cu) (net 1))
 (segment (start 144.018 108.246) (end 145.246 108.246) (width 0.6096) (layer F.Cu) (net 1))
 (segment (start 139.065 98.679) (end 139.065 99.949) (width 0.6096) (layer F.Cu) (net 1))
 (segment (start 139.744 98) (end 139.065 98.679) (width 0.6096) (layer F.Cu) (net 1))
 (segment (start 145.288 92.202) (end 145.288 95.25) (width 0.6096) (layer F.Cu) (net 1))
 (segment (start 145.796 91.694) (end 145.288 92.202) (width 0.6096) (layer F.Cu) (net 1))
 (segment (start 145.288 95.25) (end 142.538 98) (width 0.6096) (layer F.Cu) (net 1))
 (segment (start 150.114 91.694) (end 145.796 91.694) (width 0.6096) (layer F.Cu) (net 1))
 (segment (start 150.368 91.948) (end 150.114 91.694) (width 0.6096) (layer F.Cu) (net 1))
 (segment (start 142.538 98) (end 139.744 98) (width 0.6096) (layer F.Cu) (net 1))
 (segment (start 150.368 93.726) (end 150.368 91.948) (width 0.6096) (layer F.Cu) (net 1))
 (segment (start 158.284 90.678) (end 158.284 93.716) (width 0.6096) (layer F.Cu) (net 2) (status C00000))
 (segment (start 158.284 93.716) (end 158 94) (width 0.6096) (layer F.Cu) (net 2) (status C00000))
 (segment (start 142.24 103.9876) (end 143.4876 103.9876) (width 0.6096) (layer F.Cu) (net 2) (status 800000))
 (segment (start 143.4876 103.9876) (end 143.5 104) (width 0.6096) (layer F.Cu) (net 2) (status C00000))
 (segment (start 159.258 89.704) (end 158.284 90.678) (width 0.6096) (layer F.Cu) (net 2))
 (segment (start 159.258 85.852) (end 159.258 89.704) (width 0.6096) (layer F.Cu) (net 2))
 (segment (start 148.082 97.028) (end 148.548 97.028) (width 0.6096) (layer F.Cu) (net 2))
 (segment (start 148.082 93.74) (end 148.082 97.028) (width 0.6096) (layer F.Cu) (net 2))
 (segment (start 148.068 93.726) (end 148.082 93.74) (width 0.6096) (layer F.Cu) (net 2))
 (segment (start 139.782 105.704) (end 139.954 105.876) (width 0.6096) (layer F.Cu) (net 2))
 (segment (start 136.874 105.704) (end 139.782 105.704) (width 0.6096) (layer F.Cu) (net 2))
 (segment (start 139.954 101.6) (end 141.605 99.949) (width 0.6096) (layer F.Cu) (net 2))
 (segment (start 139.954 105.876) (end 139.954 101.6) (width 0.6096) (layer F.Cu) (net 2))
 (segment (start 144.018 107.146) (end 142.24 107.146) (width 0.6096) (layer F.Cu) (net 2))
 (segment (start 142.24 100.584) (end 141.605 99.949) (width 0.6096) (layer F.Cu) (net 2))
 (segment (start 142.24 107.146) (end 142.24 103.9876) (width 0.6096) (layer F.Cu) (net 2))
 (segment (start 142.24 103.9876) (end 142.24 100.584) (width 0.6096) (layer F.Cu) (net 2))
 (segment (start 147.6384 97.028) (end 148.548 97.028) (width 0.6096) (layer F.Cu) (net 2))
 (segment (start 145.972 97.028) (end 147.6384 97.028) (width 0.6096) (layer F.Cu) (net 2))
 (segment (start 143.051 99.949) (end 145.972 97.028) (width 0.6096) (layer F.Cu) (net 2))
 (segment (start 141.605 99.949) (end 143.051 99.949) (width 0.6096) (layer F.Cu) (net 2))
 (segment (start 156.718 90.212) (end 157.184 90.678) (width 0.6096) (layer F.Cu) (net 3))
 (segment (start 156.718 85.852) (end 156.718 90.212) (width 0.6096) (layer F.Cu) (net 3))
 (segment (start 154.0776 93.726) (end 152.668 93.726) (width 0.6096) (layer F.Cu) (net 3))
 (segment (start 154.9956 93.726) (end 154.0776 93.726) (width 0.6096) (layer F.Cu) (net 3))
 (segment (start 157.184 91.5376) (end 154.9956 93.726) (width 0.6096) (layer F.Cu) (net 3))
 (segment (start 157.184 90.678) (end 157.184 91.5376) (width 0.6096) (layer F.Cu) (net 3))
 (segment (start 139.932 106.954) (end 139.954 106.976) (width 0.6096) (layer F.Cu) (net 4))
 (segment (start 136.874 106.954) (end 139.932 106.954) (width 0.6096) (layer F.Cu) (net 4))
 (segment (start 133.9676 106.954) (end 132.842 105.8284) (width 0.4064) (layer F.Cu) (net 5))
 (segment (start 134.874 106.954) (end 133.9676 106.954) (width 0.4064) (layer F.Cu) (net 5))
 (segment (start 132.842 101.092) (end 133.985 99.949) (width 0.4064) (layer F.Cu) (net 5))
 (segment (start 132.842 105.8284) (end 132.842 101.092) (width 0.4064) (layer F.Cu) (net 5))
 (segment (start 133.604 108.204) (end 134.874 108.204) (width 0.4064) (layer F.Cu) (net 6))
 (segment (start 131.826 106.426) (end 133.604 108.204) (width 0.4064) (layer F.Cu) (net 6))
 (segment (start 131.826 100.076) (end 131.826 106.426) (width 0.4064) (layer F.Cu) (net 6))
 (segment (start 133.35 98.552) (end 131.826 100.076) (width 0.4064) (layer F.Cu) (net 6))
 (segment (start 135.128 98.552) (end 133.35 98.552) (width 0.4064) (layer F.Cu) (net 6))
 (segment (start 136.525 99.949) (end 135.128 98.552) (width 0.4064) (layer F.Cu) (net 6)))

